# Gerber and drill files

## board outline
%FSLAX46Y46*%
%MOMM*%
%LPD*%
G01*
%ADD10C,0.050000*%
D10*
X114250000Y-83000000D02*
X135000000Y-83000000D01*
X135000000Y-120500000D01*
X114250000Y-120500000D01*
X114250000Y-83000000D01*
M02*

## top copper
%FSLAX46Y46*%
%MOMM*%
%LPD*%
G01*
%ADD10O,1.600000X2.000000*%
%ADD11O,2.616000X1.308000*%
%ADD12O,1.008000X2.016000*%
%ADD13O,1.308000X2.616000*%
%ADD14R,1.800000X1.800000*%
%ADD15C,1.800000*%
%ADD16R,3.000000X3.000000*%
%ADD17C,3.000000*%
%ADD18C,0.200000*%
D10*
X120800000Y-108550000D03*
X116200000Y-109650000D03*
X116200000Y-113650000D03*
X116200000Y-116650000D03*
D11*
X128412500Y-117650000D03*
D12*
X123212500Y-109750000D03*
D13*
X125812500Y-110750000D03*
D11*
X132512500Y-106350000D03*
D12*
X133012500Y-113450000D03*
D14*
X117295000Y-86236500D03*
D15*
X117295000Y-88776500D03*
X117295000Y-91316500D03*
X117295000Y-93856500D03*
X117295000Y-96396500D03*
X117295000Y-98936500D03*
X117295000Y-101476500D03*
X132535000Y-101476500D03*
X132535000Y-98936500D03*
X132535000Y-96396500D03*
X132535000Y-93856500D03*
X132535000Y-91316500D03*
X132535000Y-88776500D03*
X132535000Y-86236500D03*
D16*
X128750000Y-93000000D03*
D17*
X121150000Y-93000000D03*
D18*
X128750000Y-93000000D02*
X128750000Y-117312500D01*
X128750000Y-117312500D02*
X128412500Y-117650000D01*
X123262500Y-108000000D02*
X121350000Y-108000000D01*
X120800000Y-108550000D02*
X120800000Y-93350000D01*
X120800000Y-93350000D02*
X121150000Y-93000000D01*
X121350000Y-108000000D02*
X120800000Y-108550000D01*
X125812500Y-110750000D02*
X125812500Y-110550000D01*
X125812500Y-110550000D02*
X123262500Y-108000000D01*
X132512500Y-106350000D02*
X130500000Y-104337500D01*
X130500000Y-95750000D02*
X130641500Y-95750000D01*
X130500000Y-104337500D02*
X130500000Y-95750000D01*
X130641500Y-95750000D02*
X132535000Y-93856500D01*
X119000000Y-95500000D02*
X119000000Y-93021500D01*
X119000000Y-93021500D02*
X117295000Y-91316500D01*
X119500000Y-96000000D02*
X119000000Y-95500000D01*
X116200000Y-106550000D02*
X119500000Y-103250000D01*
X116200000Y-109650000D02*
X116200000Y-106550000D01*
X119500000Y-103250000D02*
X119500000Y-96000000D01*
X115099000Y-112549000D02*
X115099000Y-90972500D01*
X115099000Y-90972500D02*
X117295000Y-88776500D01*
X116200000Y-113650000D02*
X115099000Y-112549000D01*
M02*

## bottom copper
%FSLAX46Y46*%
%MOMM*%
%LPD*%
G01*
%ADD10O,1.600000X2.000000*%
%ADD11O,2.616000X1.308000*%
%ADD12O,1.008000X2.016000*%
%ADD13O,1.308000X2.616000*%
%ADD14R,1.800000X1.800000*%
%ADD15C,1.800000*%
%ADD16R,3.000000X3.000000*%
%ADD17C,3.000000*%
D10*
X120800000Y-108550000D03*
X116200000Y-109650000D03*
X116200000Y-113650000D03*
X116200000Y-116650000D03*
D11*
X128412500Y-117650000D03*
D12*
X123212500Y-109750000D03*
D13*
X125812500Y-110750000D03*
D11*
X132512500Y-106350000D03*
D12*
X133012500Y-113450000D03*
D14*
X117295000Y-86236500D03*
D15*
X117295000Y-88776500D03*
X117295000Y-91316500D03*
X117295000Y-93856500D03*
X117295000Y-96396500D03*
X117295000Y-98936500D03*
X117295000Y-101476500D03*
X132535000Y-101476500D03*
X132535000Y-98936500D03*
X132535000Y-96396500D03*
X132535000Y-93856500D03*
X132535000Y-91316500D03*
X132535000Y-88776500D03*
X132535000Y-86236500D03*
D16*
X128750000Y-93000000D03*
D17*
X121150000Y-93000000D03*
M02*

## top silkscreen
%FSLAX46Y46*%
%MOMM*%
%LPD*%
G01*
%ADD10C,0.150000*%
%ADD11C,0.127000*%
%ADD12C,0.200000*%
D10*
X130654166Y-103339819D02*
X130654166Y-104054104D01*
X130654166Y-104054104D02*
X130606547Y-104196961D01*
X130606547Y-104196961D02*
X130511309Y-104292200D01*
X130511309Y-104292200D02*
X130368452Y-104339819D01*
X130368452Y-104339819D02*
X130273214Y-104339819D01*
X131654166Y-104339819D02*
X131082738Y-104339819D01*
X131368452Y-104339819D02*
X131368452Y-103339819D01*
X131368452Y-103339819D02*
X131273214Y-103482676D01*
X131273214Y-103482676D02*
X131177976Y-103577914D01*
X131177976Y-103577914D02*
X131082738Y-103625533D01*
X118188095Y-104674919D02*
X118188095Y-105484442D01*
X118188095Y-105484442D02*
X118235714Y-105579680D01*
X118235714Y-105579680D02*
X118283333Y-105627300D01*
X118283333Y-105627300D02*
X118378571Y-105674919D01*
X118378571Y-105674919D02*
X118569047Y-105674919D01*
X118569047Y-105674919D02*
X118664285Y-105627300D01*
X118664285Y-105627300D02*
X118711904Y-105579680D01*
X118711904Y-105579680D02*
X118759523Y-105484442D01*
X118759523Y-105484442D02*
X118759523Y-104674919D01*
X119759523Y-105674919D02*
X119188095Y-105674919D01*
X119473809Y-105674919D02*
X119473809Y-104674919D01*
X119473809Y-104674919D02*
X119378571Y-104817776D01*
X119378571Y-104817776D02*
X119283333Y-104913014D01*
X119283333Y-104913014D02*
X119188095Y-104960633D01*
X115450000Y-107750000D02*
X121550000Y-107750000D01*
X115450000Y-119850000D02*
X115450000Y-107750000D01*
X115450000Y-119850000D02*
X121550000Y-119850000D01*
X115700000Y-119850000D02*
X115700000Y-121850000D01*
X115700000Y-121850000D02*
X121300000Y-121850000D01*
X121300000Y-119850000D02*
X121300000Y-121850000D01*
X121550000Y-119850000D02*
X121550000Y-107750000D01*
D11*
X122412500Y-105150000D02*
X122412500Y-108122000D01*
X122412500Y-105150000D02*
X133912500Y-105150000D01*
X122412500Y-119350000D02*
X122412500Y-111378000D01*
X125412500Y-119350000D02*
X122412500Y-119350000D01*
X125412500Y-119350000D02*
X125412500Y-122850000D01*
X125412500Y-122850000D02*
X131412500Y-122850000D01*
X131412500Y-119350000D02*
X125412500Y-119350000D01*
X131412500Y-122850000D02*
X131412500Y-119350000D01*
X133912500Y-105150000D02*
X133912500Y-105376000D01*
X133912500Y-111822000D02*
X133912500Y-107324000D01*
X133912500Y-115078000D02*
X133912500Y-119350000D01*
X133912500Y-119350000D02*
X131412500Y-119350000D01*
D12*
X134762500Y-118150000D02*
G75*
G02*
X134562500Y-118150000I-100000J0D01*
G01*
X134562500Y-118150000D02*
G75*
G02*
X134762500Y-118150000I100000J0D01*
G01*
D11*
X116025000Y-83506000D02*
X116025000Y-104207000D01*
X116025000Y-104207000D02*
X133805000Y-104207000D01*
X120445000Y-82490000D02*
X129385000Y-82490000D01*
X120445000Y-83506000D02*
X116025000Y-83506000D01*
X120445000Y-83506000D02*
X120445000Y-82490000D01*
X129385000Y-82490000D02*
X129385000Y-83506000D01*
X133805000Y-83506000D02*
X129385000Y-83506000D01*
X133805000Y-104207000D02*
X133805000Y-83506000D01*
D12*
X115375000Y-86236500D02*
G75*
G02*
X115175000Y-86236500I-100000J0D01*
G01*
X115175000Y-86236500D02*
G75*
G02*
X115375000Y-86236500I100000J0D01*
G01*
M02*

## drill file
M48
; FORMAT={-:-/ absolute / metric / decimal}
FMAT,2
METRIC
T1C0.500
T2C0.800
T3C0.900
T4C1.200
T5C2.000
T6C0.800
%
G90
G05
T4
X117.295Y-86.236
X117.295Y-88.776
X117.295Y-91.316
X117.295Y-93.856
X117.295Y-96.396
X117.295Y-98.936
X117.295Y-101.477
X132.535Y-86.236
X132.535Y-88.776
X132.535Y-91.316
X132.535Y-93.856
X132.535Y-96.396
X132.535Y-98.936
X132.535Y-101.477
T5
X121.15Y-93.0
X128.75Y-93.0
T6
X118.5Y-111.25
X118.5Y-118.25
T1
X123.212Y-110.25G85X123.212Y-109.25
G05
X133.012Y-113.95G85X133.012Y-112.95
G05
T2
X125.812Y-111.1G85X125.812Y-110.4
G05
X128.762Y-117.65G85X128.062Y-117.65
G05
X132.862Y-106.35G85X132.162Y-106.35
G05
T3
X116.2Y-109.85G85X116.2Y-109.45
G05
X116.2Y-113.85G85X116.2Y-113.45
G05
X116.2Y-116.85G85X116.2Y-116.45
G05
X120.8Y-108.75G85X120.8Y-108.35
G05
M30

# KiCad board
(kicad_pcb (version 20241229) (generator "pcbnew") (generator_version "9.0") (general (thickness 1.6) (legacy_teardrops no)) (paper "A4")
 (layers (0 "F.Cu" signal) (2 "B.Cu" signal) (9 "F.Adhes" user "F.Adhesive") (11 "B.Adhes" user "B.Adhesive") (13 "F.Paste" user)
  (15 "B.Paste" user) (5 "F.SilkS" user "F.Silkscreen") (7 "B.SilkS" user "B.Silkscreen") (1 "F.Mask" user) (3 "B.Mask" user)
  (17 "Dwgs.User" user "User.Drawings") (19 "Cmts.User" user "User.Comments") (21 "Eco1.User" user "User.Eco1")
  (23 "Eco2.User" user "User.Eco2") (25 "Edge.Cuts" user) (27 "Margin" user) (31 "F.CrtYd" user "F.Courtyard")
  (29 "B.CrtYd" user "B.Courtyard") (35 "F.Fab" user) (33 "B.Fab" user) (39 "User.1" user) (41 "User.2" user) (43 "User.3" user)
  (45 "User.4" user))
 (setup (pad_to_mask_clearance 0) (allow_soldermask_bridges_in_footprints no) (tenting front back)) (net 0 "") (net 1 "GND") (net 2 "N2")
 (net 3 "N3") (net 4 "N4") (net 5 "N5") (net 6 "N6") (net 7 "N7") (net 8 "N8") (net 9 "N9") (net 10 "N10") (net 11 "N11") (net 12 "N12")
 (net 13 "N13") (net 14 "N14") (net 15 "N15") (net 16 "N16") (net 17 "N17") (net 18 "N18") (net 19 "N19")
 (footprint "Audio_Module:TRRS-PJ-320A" (layer "F.Cu") (at 118.5 119.85 180)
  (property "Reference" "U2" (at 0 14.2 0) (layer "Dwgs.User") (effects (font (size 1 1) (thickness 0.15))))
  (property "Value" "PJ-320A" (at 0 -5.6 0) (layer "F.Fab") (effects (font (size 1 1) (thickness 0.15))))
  (fp_line (start 3.05 12.1) (end -3.05 12.1) (stroke (width 0.15) (type solid)) (layer "F.SilkS"))
  (fp_line (start 3.05 0) (end 3.05 12.1) (stroke (width 0.15) (type solid)) (layer "F.SilkS"))
  (fp_line (start 3.05 0) (end -3.05 0) (stroke (width 0.15) (type solid)) (layer "F.SilkS"))
  (fp_line (start 2.8 0) (end 2.8 -2) (stroke (width 0.15) (type solid)) (layer "F.SilkS"))
  (fp_line (start 2.8 -2) (end -2.8 -2) (stroke (width 0.15) (type solid)) (layer "F.SilkS"))
  (fp_line (start -2.8 0) (end -2.8 -2) (stroke (width 0.15) (type solid)) (layer "F.SilkS"))
  (fp_line (start -3.05 0) (end -3.05 12.1) (stroke (width 0.15) (type solid)) (layer "F.SilkS"))
  (pad "" np_thru_hole circle (at 0 1.6 180) (size 0.8 0.8) (drill 0.8) (layers "*.Cu" "*.Mask"))
  (pad "" np_thru_hole circle (at 0 8.6 180) (size 0.8 0.8) (drill 0.8) (layers "*.Cu" "*.Mask"))
  (pad "1" thru_hole oval (at -2.3 11.3 180) (size 1.6 2) (drill oval 0.9 1.3) (layers "*.Cu" "*.Mask") (remove_unused_layers no)
   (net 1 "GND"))
  (pad "2" thru_hole oval (at 2.3 10.2 180) (size 1.6 2) (drill oval 0.9 1.3) (layers "*.Cu" "*.Mask") (remove_unused_layers no)
   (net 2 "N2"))
  (pad "3" thru_hole oval (at 2.3 6.2 180) (size 1.6 2) (drill oval 0.9 1.3) (layers "*.Cu" "*.Mask") (remove_unused_layers no) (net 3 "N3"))
  (pad "4" thru_hole oval (at 2.3 3.2 180) (size 1.6 2) (drill oval 0.9 1.3) (layers "*.Cu" "*.Mask") (remove_unused_layers no) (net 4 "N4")))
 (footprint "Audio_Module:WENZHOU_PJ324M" (layer "F.Cu") (at 128.4125 112.25 180)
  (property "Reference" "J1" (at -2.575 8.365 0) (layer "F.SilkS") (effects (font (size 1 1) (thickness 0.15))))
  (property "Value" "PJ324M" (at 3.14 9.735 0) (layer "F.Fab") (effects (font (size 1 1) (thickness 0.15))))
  (fp_line (start 6 7.1) (end 6 4.128) (stroke (width 0.127) (type solid)) (layer "F.SilkS"))
  (fp_line (start 6 7.1) (end -5.5 7.1) (stroke (width 0.127) (type solid)) (layer "F.SilkS"))
  (fp_line (start 6 -7.1) (end 6 0.872) (stroke (width 0.127) (type solid)) (layer "F.SilkS"))
  (fp_line (start 3 -7.1) (end 6 -7.1) (stroke (width 0.127) (type solid)) (layer "F.SilkS"))
  (fp_line (start 3 -7.1) (end 3 -10.6) (stroke (width 0.127) (type solid)) (layer "F.SilkS"))
  (fp_line (start 3 -10.6) (end -3 -10.6) (stroke (width 0.127) (type solid)) (layer "F.SilkS"))
  (fp_line (start -3 -7.1) (end 3 -7.1) (stroke (width 0.127) (type solid)) (layer "F.SilkS"))
  (fp_line (start -3 -10.6) (end -3 -7.1) (stroke (width 0.127) (type solid)) (layer "F.SilkS"))
  (fp_line (start -5.5 7.1) (end -5.5 6.874) (stroke (width 0.127) (type solid)) (layer "F.SilkS"))
  (fp_line (start -5.5 0.428) (end -5.5 4.926) (stroke (width 0.127) (type solid)) (layer "F.SilkS"))
  (fp_line (start -5.5 -2.828) (end -5.5 -7.1) (stroke (width 0.127) (type solid)) (layer "F.SilkS"))
  (fp_line (start -5.5 -7.1) (end -3 -7.1) (stroke (width 0.127) (type solid)) (layer "F.SilkS"))
  (fp_circle (center -6.25 -5.9) (end -6.15 -5.9) (stroke (width 0.2) (type solid)) (fill no) (layer "F.SilkS"))
  (pad "1" thru_hole oval (at 0 -5.4 180) (size 2.616 1.308) (drill oval 1.5 0.8) (layers "*.Cu" "*.Mask") (remove_unused_layers no)
   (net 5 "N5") (solder_mask_margin 0.102))
  (pad "2" thru_hole oval (at 5.2 2.5 180) (size 1.008 2.016) (drill oval 0.5 1.5) (layers "*.Cu" "*.Mask") (remove_unused_layers no)
   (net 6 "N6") (solder_mask_margin 0.102))
  (pad "3" thru_hole oval (at 2.6 1.5 180) (size 1.308 2.616) (drill oval 0.8 1.5) (layers "*.Cu" "*.Mask") (remove_unused_layers no)
   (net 1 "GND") (solder_mask_margin 0.102))
  (pad "4" thru_hole oval (at -4.1 5.9 180) (size 2.616 1.308) (drill oval 1.5 0.8) (layers "*.Cu" "*.Mask") (remove_unused_layers no)
   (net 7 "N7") (solder_mask_margin 0.102))
  (pad "5" thru_hole oval (at -4.6 -1.2 180) (size 1.008 2.016) (drill oval 0.5 1.5) (layers "*.Cu" "*.Mask") (remove_unused_layers no)
   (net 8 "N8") (solder_mask_margin 0.102)))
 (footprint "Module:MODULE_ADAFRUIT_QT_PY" (layer "F.Cu") (at 124.915 93.8565)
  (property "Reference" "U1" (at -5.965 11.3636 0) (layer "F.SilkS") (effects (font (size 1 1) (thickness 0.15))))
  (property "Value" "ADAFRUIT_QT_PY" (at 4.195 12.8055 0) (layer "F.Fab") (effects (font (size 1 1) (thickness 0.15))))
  (fp_line (start -8.89 -10.3505) (end -8.89 10.3505) (stroke (width 0.127) (type solid)) (layer "F.SilkS"))
  (fp_line (start -8.89 10.3505) (end 8.89 10.3505) (stroke (width 0.127) (type solid)) (layer "F.SilkS"))
  (fp_line (start -4.47 -11.3665) (end 4.47 -11.3665) (stroke (width 0.127) (type solid)) (layer "F.SilkS"))
  (fp_line (start -4.47 -10.3505) (end -8.89 -10.3505) (stroke (width 0.127) (type solid)) (layer "F.SilkS"))
  (fp_line (start -4.47 -10.3505) (end -4.47 -11.3665) (stroke (width 0.127) (type solid)) (layer "F.SilkS"))
  (fp_line (start 4.47 -11.3665) (end 4.47 -10.3505) (stroke (width 0.127) (type solid)) (layer "F.SilkS"))
  (fp_line (start 8.89 -10.3505) (end 4.47 -10.3505) (stroke (width 0.127) (type solid)) (layer "F.SilkS"))
  (fp_line (start 8.89 10.3505) (end 8.89 -10.3505) (stroke (width 0.127) (type solid)) (layer "F.SilkS"))
  (fp_circle (center -9.64 -7.62) (end -9.54 -7.62) (stroke (width 0.2) (type solid)) (fill no) (layer "F.SilkS"))
  (pad "1" thru_hole rect (at -7.62 -7.62) (size 1.8 1.8) (drill 1.2) (layers "*.Cu" "*.Mask") (remove_unused_layers no) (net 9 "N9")
   (solder_mask_margin 0.102))
  (pad "2" thru_hole circle (at -7.62 -5.08) (size 1.8 1.8) (drill 1.2) (layers "*.Cu" "*.Mask") (remove_unused_layers no) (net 3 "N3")
   (solder_mask_margin 0.102))
  (pad "3" thru_hole circle (at -7.62 -2.54) (size 1.8 1.8) (drill 1.2) (layers "*.Cu" "*.Mask") (remove_unused_layers no) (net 2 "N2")
   (solder_mask_margin 0.102))
  (pad "4" thru_hole circle (at -7.62 0) (size 1.8 1.8) (drill 1.2) (layers "*.Cu" "*.Mask") (remove_unused_layers no) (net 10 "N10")
   (solder_mask_margin 0.102))
  (pad "5" thru_hole circle (at -7.62 2.54) (size 1.8 1.8) (drill 1.2) (layers "*.Cu" "*.Mask") (remove_unused_layers no) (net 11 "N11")
   (solder_mask_margin 0.102))
  (pad "6" thru_hole circle (at -7.62 5.08) (size 1.8 1.8) (drill 1.2) (layers "*.Cu" "*.Mask") (remove_unused_layers no) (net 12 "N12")
   (solder_mask_margin 0.102))
  (pad "7" thru_hole circle (at -7.62 7.62) (size 1.8 1.8) (drill 1.2) (layers "*.Cu" "*.Mask") (remove_unused_layers no) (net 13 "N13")
   (solder_mask_margin 0.102))
  (pad "8" thru_hole circle (at 7.62 7.62) (size 1.8 1.8) (drill 1.2) (layers "*.Cu" "*.Mask") (remove_unused_layers no) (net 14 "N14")
   (solder_mask_margin 0.102))
  (pad "9" thru_hole circle (at 7.62 5.08) (size 1.8 1.8) (drill 1.2) (layers "*.Cu" "*.Mask") (remove_unused_layers no) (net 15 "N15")
   (solder_mask_margin 0.102))
  (pad "10" thru_hole circle (at 7.62 2.54) (size 1.8 1.8) (drill 1.2) (layers "*.Cu" "*.Mask") (remove_unused_layers no) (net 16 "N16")
   (solder_mask_margin 0.102))
  (pad "11" thru_hole circle (at 7.62 0) (size 1.8 1.8) (drill 1.2) (layers "*.Cu" "*.Mask") (remove_unused_layers no) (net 7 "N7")
   (solder_mask_margin 0.102))
  (pad "12" thru_hole circle (at 7.62 -2.54) (size 1.8 1.8) (drill 1.2) (layers "*.Cu" "*.Mask") (remove_unused_layers no) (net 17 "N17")
   (solder_mask_margin 0.102))
  (pad "13" thru_hole circle (at 7.62 -5.08) (size 1.8 1.8) (drill 1.2) (layers "*.Cu" "*.Mask") (remove_unused_layers no) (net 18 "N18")
   (solder_mask_margin 0.102))
  (pad "14" thru_hole circle (at 7.62 -7.62) (size 1.8 1.8) (drill 1.2) (layers "*.Cu" "*.Mask") (remove_unused_layers no) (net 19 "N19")
   (solder_mask_margin 0.102)))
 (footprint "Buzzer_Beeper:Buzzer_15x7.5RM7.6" (layer "B.Cu") (at 128.75 93 180)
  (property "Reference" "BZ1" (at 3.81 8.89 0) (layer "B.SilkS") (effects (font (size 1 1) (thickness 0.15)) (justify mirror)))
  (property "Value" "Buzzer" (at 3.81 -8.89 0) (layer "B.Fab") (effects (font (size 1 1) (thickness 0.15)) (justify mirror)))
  (pad "1" thru_hole rect (at 0 0 180) (size 3 3) (drill 2) (layers "*.Cu" "*.Mask") (remove_unused_layers no) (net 5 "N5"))
  (pad "2" thru_hole circle (at 7.6 0 180) (size 3 3) (drill 2) (layers "*.Cu" "*.Mask") (remove_unused_layers no) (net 1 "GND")))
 (gr_rect (start 114.25 83) (end 135 120.5) (stroke (width 0.05) (type default)) (fill no) (layer "Edge.Cuts"))
 (segment (start 128.75 93) (end 128.75 117.3125) (width 0.2) (layer "F.Cu") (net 5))
 (segment (start 128.75 117.3125) (end 128.4125 117.65) (width 0.2) (layer "F.Cu") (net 5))
 (segment (start 123.2625 108) (end 121.35 108) (width 0.2) (layer "F.Cu") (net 1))
 (segment (start 120.8 108.55) (end 120.8 93.35) (width 0.2) (layer "F.Cu") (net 1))
 (segment (start 120.8 93.35) (end 121.15 93) (width 0.2) (layer "F.Cu") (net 1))
 (segment (start 121.35 108) (end 120.8 108.55) (width 0.2) (layer "F.Cu") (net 1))
 (segment (start 125.8125 110.75) (end 125.8125 110.55) (width 0.2) (layer "F.Cu") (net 1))
 (segment (start 125.8125 110.55) (end 123.2625 108) (width 0.2) (layer "F.Cu") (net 1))
 (segment (start 132.5125 106.35) (end 130.5 104.3375) (width 0.2) (layer "F.Cu") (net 7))
 (segment (start 130.5 95.75) (end 130.6415 95.75) (width 0.2) (layer "F.Cu") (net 7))
 (segment (start 130.5 104.3375) (end 130.5 95.75) (width 0.2) (layer "F.Cu") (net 7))
 (segment (start 130.6415 95.75) (end 132.535 93.8565) (width 0.2) (layer "F.Cu") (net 7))
 (segment (start 119 95.5) (end 119 93.0215) (width 0.2) (layer "F.Cu") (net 2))
 (segment (start 119 93.0215) (end 117.295 91.3165) (width 0.2) (layer "F.Cu") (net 2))
 (segment (start 119.5 96) (end 119 95.5) (width 0.2) (layer "F.Cu") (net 2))
 (segment (start 116.2 106.55) (end 119.5 103.25) (width 0.2) (layer "F.Cu") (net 2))
 (segment (start 116.2 109.65) (end 116.2 106.55) (width 0.2) (layer "F.Cu") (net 2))
 (segment (start 119.5 103.25) (end 119.5 96) (width 0.2) (layer "F.Cu") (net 2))
 (segment (start 115.099 112.549) (end 115.099 90.9725) (width 0.2) (layer "F.Cu") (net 3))
 (segment (start 115.099 90.9725) (end 117.295 88.7765) (width 0.2) (layer "F.Cu") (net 3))
 (segment (start 116.2 113.65) (end 115.099 112.549) (width 0.2) (layer "F.Cu") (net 3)))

